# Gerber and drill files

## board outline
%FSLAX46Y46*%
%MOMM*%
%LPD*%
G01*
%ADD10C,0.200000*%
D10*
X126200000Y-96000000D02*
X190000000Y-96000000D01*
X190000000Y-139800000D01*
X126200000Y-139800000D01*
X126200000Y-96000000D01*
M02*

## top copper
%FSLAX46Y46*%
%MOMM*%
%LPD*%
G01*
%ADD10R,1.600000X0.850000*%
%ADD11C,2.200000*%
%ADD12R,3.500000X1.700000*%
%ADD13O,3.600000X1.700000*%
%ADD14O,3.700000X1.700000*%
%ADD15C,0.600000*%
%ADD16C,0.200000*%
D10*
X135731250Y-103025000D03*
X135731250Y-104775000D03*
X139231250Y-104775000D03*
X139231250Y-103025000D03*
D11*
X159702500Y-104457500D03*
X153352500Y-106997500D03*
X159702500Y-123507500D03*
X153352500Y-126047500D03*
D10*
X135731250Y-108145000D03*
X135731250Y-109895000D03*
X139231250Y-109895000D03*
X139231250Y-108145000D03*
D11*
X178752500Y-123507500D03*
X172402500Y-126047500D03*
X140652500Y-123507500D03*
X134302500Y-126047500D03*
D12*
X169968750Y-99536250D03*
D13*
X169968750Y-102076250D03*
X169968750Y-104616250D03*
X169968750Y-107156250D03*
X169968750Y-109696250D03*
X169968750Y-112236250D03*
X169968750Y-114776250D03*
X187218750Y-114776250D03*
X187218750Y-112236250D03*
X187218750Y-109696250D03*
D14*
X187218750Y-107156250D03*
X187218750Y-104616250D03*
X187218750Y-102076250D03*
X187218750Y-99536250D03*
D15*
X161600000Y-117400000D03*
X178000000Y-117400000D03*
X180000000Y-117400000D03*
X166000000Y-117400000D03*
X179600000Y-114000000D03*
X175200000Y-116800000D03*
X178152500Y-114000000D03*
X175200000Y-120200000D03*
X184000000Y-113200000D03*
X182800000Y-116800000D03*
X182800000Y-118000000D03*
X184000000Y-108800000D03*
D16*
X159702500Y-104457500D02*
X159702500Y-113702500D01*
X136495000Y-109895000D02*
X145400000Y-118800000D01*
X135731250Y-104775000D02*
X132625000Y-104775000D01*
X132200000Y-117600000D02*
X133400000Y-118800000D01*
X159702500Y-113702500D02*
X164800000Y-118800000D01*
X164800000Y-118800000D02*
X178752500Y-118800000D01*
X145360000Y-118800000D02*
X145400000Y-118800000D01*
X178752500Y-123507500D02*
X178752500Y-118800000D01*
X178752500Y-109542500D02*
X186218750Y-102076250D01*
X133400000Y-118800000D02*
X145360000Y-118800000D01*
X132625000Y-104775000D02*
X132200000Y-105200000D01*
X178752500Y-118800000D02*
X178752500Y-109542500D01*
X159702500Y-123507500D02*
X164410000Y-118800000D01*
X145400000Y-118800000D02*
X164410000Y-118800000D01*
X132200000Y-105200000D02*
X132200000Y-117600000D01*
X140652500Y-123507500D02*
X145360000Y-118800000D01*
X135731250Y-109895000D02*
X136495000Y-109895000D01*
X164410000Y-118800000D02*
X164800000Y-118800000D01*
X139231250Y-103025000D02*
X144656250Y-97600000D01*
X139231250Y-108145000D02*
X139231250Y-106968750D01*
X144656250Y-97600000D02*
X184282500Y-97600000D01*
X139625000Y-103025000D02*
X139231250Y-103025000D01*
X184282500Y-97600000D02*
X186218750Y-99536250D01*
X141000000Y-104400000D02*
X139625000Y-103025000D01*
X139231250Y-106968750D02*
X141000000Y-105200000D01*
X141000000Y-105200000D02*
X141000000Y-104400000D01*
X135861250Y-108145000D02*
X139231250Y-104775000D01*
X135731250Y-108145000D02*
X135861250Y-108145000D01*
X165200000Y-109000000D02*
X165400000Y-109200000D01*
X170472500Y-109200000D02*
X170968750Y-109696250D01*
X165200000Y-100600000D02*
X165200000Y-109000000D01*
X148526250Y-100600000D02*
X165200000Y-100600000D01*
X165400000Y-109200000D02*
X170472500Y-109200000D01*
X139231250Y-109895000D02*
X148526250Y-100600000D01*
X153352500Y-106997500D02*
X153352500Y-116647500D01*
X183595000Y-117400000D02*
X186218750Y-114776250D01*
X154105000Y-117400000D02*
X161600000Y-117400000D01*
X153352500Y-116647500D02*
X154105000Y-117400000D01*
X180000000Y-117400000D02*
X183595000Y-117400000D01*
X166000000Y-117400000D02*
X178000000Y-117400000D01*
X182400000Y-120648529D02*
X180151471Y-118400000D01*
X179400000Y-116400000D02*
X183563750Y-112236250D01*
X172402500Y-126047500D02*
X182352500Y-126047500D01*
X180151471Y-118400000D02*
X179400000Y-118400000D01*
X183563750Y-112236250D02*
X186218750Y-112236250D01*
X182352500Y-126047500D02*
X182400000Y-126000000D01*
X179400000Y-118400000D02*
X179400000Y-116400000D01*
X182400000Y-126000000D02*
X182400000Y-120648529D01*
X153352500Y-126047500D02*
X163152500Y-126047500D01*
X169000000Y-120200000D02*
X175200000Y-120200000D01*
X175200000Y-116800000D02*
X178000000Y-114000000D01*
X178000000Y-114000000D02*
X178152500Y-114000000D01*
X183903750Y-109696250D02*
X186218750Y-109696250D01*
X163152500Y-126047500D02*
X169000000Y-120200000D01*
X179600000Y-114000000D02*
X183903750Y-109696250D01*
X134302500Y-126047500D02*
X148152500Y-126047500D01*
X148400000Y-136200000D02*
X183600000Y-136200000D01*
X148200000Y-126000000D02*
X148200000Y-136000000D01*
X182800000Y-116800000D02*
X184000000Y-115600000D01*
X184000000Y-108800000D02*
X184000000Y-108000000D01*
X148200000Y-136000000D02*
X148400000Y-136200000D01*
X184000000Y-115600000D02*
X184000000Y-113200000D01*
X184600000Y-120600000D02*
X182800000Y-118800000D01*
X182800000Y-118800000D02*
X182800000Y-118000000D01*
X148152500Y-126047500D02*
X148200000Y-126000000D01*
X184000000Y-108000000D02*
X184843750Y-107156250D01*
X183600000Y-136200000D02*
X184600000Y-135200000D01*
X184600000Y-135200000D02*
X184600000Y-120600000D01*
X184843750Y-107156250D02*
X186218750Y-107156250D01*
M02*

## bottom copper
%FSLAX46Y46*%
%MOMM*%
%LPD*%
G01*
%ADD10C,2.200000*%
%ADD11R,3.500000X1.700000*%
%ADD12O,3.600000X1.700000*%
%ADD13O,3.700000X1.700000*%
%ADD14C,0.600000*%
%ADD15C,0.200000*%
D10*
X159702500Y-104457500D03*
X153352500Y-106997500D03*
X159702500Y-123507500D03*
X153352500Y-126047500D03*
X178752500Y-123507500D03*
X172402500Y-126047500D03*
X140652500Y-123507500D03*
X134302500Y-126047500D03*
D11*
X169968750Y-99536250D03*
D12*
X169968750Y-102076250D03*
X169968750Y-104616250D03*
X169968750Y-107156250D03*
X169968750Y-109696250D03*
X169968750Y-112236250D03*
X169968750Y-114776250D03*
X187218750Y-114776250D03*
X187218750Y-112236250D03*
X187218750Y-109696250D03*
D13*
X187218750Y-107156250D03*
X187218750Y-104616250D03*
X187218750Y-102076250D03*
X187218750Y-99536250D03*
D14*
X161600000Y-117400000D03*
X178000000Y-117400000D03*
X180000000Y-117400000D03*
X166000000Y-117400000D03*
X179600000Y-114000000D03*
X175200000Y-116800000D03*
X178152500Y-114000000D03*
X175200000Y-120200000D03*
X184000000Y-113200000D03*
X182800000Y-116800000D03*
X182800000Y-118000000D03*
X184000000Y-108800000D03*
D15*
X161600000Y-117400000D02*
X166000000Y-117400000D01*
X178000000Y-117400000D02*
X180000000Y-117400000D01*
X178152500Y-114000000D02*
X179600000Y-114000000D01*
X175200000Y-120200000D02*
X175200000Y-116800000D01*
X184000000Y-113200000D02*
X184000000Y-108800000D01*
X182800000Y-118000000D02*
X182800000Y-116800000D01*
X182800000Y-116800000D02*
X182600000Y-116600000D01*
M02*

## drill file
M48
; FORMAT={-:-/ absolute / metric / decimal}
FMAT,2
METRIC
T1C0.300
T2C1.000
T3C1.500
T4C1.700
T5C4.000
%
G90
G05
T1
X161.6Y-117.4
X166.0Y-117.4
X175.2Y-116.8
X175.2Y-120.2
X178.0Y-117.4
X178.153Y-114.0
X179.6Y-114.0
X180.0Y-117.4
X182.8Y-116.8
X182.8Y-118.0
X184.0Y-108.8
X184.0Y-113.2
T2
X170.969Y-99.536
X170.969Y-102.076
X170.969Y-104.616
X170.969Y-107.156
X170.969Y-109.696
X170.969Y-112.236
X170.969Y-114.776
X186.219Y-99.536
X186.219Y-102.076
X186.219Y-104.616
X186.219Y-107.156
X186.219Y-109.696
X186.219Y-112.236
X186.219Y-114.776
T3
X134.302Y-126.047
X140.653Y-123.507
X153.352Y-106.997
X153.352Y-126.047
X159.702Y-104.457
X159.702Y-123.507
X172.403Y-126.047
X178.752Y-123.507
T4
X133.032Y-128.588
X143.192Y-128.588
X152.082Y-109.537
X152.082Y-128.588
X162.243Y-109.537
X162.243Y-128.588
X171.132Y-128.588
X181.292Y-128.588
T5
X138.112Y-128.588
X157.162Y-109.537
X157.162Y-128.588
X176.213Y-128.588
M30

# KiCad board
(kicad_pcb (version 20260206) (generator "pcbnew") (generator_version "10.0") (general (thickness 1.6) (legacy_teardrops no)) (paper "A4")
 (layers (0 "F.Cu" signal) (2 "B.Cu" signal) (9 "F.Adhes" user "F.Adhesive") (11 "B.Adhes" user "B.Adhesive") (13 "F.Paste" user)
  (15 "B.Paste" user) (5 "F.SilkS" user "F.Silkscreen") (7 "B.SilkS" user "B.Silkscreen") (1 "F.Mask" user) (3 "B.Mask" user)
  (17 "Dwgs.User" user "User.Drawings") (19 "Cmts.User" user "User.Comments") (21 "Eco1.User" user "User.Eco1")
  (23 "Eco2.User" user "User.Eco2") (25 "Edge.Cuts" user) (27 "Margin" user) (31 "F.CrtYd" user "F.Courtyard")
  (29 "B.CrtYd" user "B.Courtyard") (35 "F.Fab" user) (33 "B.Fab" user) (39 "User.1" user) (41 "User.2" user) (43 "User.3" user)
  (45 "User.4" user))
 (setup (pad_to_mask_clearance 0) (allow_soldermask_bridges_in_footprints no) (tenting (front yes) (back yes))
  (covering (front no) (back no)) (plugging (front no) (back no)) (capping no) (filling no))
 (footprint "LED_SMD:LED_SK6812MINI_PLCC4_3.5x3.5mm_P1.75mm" (layer "F.Cu") (at 137.48125 103.9)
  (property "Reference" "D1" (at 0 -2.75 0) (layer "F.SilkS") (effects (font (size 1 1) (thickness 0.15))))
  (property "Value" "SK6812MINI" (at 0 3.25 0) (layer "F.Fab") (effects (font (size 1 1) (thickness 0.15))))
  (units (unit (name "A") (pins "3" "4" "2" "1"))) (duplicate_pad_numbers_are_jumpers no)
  (pad "1" smd rect (at -1.75 -0.875) (size 1.6 0.85) (layers "F.Cu" "F.Mask" "F.Paste") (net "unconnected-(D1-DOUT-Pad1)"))
  (pad "2" smd rect (at -1.75 0.875) (size 1.6 0.85) (layers "F.Cu" "F.Mask" "F.Paste") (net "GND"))
  (pad "3" smd rect (at 1.75 0.875) (size 1.6 0.85) (layers "F.Cu" "F.Mask" "F.Paste") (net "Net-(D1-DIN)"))
  (pad "4" smd rect (at 1.75 -0.875) (size 1.6 0.85) (layers "F.Cu" "F.Mask" "F.Paste") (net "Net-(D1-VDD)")))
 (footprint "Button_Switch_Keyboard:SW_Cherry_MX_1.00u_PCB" (layer "F.Cu") (at 159.7025 104.4575)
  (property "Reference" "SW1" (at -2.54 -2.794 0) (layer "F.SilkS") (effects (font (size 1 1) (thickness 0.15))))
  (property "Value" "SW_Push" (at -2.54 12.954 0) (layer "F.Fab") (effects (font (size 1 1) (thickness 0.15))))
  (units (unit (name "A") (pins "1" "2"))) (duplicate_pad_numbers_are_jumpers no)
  (pad "" np_thru_hole circle (at -7.62 5.08) (size 1.7 1.7) (drill 1.7) (layers "*.Cu" "*.Mask"))
  (pad "" np_thru_hole circle (at -2.54 5.08) (size 4 4) (drill 4) (layers "*.Cu" "*.Mask"))
  (pad "" np_thru_hole circle (at 2.54 5.08) (size 1.7 1.7) (drill 1.7) (layers "*.Cu" "*.Mask"))
  (pad "1" thru_hole circle (at 0 0) (size 2.2 2.2) (drill 1.5) (layers "*.Cu" "*.Mask") (remove_unused_layers no) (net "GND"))
  (pad "2" thru_hole circle (at -6.35 2.54) (size 2.2 2.2) (drill 1.5) (layers "*.Cu" "*.Mask") (remove_unused_layers no)
   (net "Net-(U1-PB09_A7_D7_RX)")))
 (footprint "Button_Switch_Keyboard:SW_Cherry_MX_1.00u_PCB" (layer "F.Cu") (at 159.7025 123.5075)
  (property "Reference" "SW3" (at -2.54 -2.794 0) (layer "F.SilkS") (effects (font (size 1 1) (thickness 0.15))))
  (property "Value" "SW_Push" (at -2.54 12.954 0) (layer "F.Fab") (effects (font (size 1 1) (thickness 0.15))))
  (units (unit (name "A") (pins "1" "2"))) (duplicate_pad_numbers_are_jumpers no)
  (pad "" np_thru_hole circle (at -7.62 5.08) (size 1.7 1.7) (drill 1.7) (layers "*.Cu" "*.Mask"))
  (pad "" np_thru_hole circle (at -2.54 5.08) (size 4 4) (drill 4) (layers "*.Cu" "*.Mask"))
  (pad "" np_thru_hole circle (at 2.54 5.08) (size 1.7 1.7) (drill 1.7) (layers "*.Cu" "*.Mask"))
  (pad "1" thru_hole circle (at 0 0) (size 2.2 2.2) (drill 1.5) (layers "*.Cu" "*.Mask") (remove_unused_layers no) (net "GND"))
  (pad "2" thru_hole circle (at -6.35 2.54) (size 2.2 2.2) (drill 1.5) (layers "*.Cu" "*.Mask") (remove_unused_layers no)
   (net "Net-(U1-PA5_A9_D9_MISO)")))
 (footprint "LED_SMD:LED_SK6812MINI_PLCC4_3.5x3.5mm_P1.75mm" (layer "F.Cu") (at 137.48125 109.02)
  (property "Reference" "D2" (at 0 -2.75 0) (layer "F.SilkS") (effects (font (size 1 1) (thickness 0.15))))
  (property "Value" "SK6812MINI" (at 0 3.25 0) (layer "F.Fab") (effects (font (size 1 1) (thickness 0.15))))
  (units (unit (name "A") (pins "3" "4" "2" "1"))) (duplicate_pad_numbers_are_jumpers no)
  (pad "1" smd rect (at -1.75 -0.875) (size 1.6 0.85) (layers "F.Cu" "F.Mask" "F.Paste") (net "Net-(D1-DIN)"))
  (pad "2" smd rect (at -1.75 0.875) (size 1.6 0.85) (layers "F.Cu" "F.Mask" "F.Paste") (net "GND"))
  (pad "3" smd rect (at 1.75 0.875) (size 1.6 0.85) (layers "F.Cu" "F.Mask" "F.Paste") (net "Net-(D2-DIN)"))
  (pad "4" smd rect (at 1.75 -0.875) (size 1.6 0.85) (layers "F.Cu" "F.Mask" "F.Paste") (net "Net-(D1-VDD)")))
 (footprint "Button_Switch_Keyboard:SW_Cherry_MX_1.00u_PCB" (layer "F.Cu") (at 178.7525 123.5075)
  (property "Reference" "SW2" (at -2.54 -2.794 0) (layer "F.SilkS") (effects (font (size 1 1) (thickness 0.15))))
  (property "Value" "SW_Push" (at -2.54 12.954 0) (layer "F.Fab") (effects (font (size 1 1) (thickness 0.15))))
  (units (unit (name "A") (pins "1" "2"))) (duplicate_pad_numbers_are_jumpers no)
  (pad "" np_thru_hole circle (at -7.62 5.08) (size 1.7 1.7) (drill 1.7) (layers "*.Cu" "*.Mask"))
  (pad "" np_thru_hole circle (at -2.54 5.08) (size 4 4) (drill 4) (layers "*.Cu" "*.Mask"))
  (pad "" np_thru_hole circle (at 2.54 5.08) (size 1.7 1.7) (drill 1.7) (layers "*.Cu" "*.Mask"))
  (pad "1" thru_hole circle (at 0 0) (size 2.2 2.2) (drill 1.5) (layers "*.Cu" "*.Mask") (remove_unused_layers no) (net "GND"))
  (pad "2" thru_hole circle (at -6.35 2.54) (size 2.2 2.2) (drill 1.5) (layers "*.Cu" "*.Mask") (remove_unused_layers no)
   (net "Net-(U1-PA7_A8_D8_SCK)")))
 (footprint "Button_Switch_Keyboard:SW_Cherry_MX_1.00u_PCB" (layer "F.Cu") (at 140.6525 123.5075)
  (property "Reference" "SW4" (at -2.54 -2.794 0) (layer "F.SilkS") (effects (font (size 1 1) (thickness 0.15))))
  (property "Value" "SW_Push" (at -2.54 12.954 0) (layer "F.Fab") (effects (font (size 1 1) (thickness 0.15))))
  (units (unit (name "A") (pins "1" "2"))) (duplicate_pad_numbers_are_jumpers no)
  (pad "" np_thru_hole circle (at -7.62 5.08) (size 1.7 1.7) (drill 1.7) (layers "*.Cu" "*.Mask"))
  (pad "" np_thru_hole circle (at -2.54 5.08) (size 4 4) (drill 4) (layers "*.Cu" "*.Mask"))
  (pad "" np_thru_hole circle (at 2.54 5.08) (size 1.7 1.7) (drill 1.7) (layers "*.Cu" "*.Mask"))
  (pad "1" thru_hole circle (at 0 0) (size 2.2 2.2) (drill 1.5) (layers "*.Cu" "*.Mask") (remove_unused_layers no) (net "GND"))
  (pad "2" thru_hole circle (at -6.35 2.54) (size 2.2 2.2) (drill 1.5) (layers "*.Cu" "*.Mask") (remove_unused_layers no)
   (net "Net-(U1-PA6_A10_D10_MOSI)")))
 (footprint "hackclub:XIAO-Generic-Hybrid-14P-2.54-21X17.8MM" (layer "F.Cu") (at 178.59375 107.15625)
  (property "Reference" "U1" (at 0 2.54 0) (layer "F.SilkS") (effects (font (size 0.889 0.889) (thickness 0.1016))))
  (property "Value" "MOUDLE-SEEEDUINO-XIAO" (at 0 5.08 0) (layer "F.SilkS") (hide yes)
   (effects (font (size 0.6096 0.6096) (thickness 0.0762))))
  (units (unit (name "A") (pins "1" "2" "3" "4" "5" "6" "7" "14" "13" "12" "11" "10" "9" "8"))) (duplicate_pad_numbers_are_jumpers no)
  (pad "1" thru_hole rect (at -7.625 -7.62) (size 3.5 1.7) (drill 1 (offset -1 0)) (layers "*.Cu" "*.Mask") (remove_unused_layers no)
   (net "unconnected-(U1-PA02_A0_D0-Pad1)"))
  (pad "2" thru_hole oval (at -7.625 -5.08) (size 3.6 1.7) (drill 1 (offset -1 0)) (layers "*.Cu" "*.Mask") (remove_unused_layers no)
   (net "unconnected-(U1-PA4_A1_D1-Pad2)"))
  (pad "3" thru_hole oval (at -7.625 -2.54) (size 3.6 1.7) (drill 1 (offset -1 0)) (layers "*.Cu" "*.Mask") (remove_unused_layers no)
   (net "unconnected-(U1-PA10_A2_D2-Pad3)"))
  (pad "4" thru_hole oval (at -7.625 0) (size 3.6 1.7) (drill 1 (offset -1 0)) (layers "*.Cu" "*.Mask") (remove_unused_layers no)
   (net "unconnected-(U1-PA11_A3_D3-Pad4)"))
  (pad "5" thru_hole oval (at -7.625 2.54) (size 3.6 1.7) (drill 1 (offset -1 0)) (layers "*.Cu" "*.Mask") (remove_unused_layers no)
   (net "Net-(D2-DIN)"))
  (pad "6" thru_hole oval (at -7.625 5.08 180) (size 3.6 1.7) (drill 1 (offset 1 0)) (layers "*.Cu" "*.Mask") (remove_unused_layers no)
   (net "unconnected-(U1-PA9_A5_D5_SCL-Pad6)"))
  (pad "7" thru_hole oval (at -7.625 7.62) (size 3.6 1.7) (drill 1 (offset -1 0)) (layers "*.Cu" "*.Mask") (remove_unused_layers no)
   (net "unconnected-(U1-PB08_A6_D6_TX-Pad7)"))
  (pad "8" thru_hole oval (at 7.625 7.62) (size 3.6 1.7) (drill 1 (offset 1 0)) (layers "*.Cu" "*.Mask") (remove_unused_layers no)
   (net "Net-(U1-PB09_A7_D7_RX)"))
  (pad "9" thru_hole oval (at 7.625 5.08) (size 3.6 1.7) (drill 1 (offset 1 0)) (layers "*.Cu" "*.Mask") (remove_unused_layers no)
   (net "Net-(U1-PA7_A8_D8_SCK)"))
  (pad "10" thru_hole oval (at 7.625 2.54) (size 3.6 1.7) (drill 1 (offset 1 0)) (layers "*.Cu" "*.Mask") (remove_unused_layers no)
   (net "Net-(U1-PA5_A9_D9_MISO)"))
  (pad "11" thru_hole oval (at 7.625 0) (size 3.7 1.7) (drill 1 (offset 1 0)) (layers "*.Cu" "*.Mask") (remove_unused_layers no)
   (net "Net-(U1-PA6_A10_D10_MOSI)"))
  (pad "12" thru_hole oval (at 7.625 -2.54) (size 3.7 1.7) (drill 1 (offset 1 0)) (layers "*.Cu" "*.Mask") (remove_unused_layers no)
   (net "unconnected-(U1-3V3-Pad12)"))
  (pad "13" thru_hole oval (at 7.625 -5.08) (size 3.7 1.7) (drill 1 (offset 1 0)) (layers "*.Cu" "*.Mask") (remove_unused_layers no)
   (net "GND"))
  (pad "14" thru_hole oval (at 7.625 -7.62) (size 3.7 1.7) (drill 1 (offset 1 0)) (layers "*.Cu" "*.Mask") (remove_unused_layers no)
   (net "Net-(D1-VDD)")))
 (gr_rect (start 126.2 96) (end 190 139.8) (stroke (width 0.2) (type solid)) (fill no) (layer "Edge.Cuts"))
 (segment (start 159.7025 104.4575) (end 159.7025 113.7025) (width 0.2) (layer "F.Cu") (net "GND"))
 (segment (start 136.495 109.895) (end 145.4 118.8) (width 0.2) (layer "F.Cu") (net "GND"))
 (segment (start 135.73125 104.775) (end 132.625 104.775) (width 0.2) (layer "F.Cu") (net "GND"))
 (segment (start 132.2 117.6) (end 133.4 118.8) (width 0.2) (layer "F.Cu") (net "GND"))
 (segment (start 159.7025 113.7025) (end 164.8 118.8) (width 0.2) (layer "F.Cu") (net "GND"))
 (segment (start 164.8 118.8) (end 178.7525 118.8) (width 0.2) (layer "F.Cu") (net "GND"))
 (segment (start 145.36 118.8) (end 145.4 118.8) (width 0.2) (layer "F.Cu") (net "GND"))
 (segment (start 178.7525 123.5075) (end 178.7525 118.8) (width 0.2) (layer "F.Cu") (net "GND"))
 (segment (start 178.7525 109.5425) (end 186.21875 102.07625) (width 0.2) (layer "F.Cu") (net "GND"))
 (segment (start 133.4 118.8) (end 145.36 118.8) (width 0.2) (layer "F.Cu") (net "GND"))
 (segment (start 132.625 104.775) (end 132.2 105.2) (width 0.2) (layer "F.Cu") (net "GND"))
 (segment (start 178.7525 118.8) (end 178.7525 109.5425) (width 0.2) (layer "F.Cu") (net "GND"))
 (segment (start 159.7025 123.5075) (end 164.41 118.8) (width 0.2) (layer "F.Cu") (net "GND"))
 (segment (start 145.4 118.8) (end 164.41 118.8) (width 0.2) (layer "F.Cu") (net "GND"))
 (segment (start 132.2 105.2) (end 132.2 117.6) (width 0.2) (layer "F.Cu") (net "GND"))
 (segment (start 140.6525 123.5075) (end 145.36 118.8) (width 0.2) (layer "F.Cu") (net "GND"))
 (segment (start 135.73125 109.895) (end 136.495 109.895) (width 0.2) (layer "F.Cu") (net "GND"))
 (segment (start 164.41 118.8) (end 164.8 118.8) (width 0.2) (layer "F.Cu") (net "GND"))
 (segment (start 139.23125 103.025) (end 144.65625 97.6) (width 0.2) (layer "F.Cu") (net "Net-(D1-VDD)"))
 (segment (start 139.23125 108.145) (end 139.23125 106.96875) (width 0.2) (layer "F.Cu") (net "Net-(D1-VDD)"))
 (segment (start 144.65625 97.6) (end 184.2825 97.6) (width 0.2) (layer "F.Cu") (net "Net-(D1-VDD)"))
 (segment (start 139.625 103.025) (end 139.23125 103.025) (width 0.2) (layer "F.Cu") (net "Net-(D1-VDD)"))
 (segment (start 184.2825 97.6) (end 186.21875 99.53625) (width 0.2) (layer "F.Cu") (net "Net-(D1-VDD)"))
 (segment (start 141 104.4) (end 139.625 103.025) (width 0.2) (layer "F.Cu") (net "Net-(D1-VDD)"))
 (segment (start 139.23125 106.96875) (end 141 105.2) (width 0.2) (layer "F.Cu") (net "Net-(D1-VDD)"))
 (segment (start 141 105.2) (end 141 104.4) (width 0.2) (layer "F.Cu") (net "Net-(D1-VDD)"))
 (segment (start 135.86125 108.145) (end 139.23125 104.775) (width 0.2) (layer "F.Cu") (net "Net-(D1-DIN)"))
 (segment (start 135.73125 108.145) (end 135.86125 108.145) (width 0.2) (layer "F.Cu") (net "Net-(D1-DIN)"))
 (segment (start 165.2 109) (end 165.4 109.2) (width 0.2) (layer "F.Cu") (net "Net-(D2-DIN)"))
 (segment (start 170.4725 109.2) (end 170.96875 109.69625) (width 0.2) (layer "F.Cu") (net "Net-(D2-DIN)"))
 (segment (start 165.2 100.6) (end 165.2 109) (width 0.2) (layer "F.Cu") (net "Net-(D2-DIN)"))
 (segment (start 148.52625 100.6) (end 165.2 100.6) (width 0.2) (layer "F.Cu") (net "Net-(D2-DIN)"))
 (segment (start 165.4 109.2) (end 170.4725 109.2) (width 0.2) (layer "F.Cu") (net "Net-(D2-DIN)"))
 (segment (start 139.23125 109.895) (end 148.52625 100.6) (width 0.2) (layer "F.Cu") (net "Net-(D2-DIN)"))
 (segment (start 153.3525 106.9975) (end 153.3525 116.6475) (width 0.2) (layer "F.Cu") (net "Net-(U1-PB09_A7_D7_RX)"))
 (segment (start 183.595 117.4) (end 186.21875 114.77625) (width 0.2) (layer "F.Cu") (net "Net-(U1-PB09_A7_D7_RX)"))
 (segment (start 154.105 117.4) (end 161.6 117.4) (width 0.2) (layer "F.Cu") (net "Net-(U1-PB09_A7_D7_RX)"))
 (segment (start 153.3525 116.6475) (end 154.105 117.4) (width 0.2) (layer "F.Cu") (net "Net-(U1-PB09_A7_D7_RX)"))
 (segment (start 180 117.4) (end 183.595 117.4) (width 0.2) (layer "F.Cu") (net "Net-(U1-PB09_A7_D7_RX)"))
 (segment (start 166 117.4) (end 178 117.4) (width 0.2) (layer "F.Cu") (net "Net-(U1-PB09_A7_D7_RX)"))
 (via (at 161.6 117.4) (size 0.6) (drill 0.3) (layers "F.Cu" "B.Cu") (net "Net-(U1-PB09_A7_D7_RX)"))
 (via (at 178 117.4) (size 0.6) (drill 0.3) (layers "F.Cu" "B.Cu") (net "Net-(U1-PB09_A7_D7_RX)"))
 (via (at 180 117.4) (size 0.6) (drill 0.3) (layers "F.Cu" "B.Cu") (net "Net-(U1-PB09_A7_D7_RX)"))
 (via (at 166 117.4) (size 0.6) (drill 0.3) (layers "F.Cu" "B.Cu") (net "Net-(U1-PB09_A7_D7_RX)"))
 (segment (start 161.6 117.4) (end 166 117.4) (width 0.2) (layer "B.Cu") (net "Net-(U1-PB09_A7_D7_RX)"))
 (segment (start 178 117.4) (end 180 117.4) (width 0.2) (layer "B.Cu") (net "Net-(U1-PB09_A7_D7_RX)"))
 (segment (start 182.4 120.648529) (end 180.151471 118.4) (width 0.2) (layer "F.Cu") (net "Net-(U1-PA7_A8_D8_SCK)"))
 (segment (start 179.4 116.4) (end 183.56375 112.23625) (width 0.2) (layer "F.Cu") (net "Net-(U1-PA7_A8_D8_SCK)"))
 (segment (start 172.4025 126.0475) (end 182.3525 126.0475) (width 0.2) (layer "F.Cu") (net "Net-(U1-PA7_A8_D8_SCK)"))
 (segment (start 180.151471 118.4) (end 179.4 118.4) (width 0.2) (layer "F.Cu") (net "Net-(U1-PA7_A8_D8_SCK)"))
 (segment (start 183.56375 112.23625) (end 186.21875 112.23625) (width 0.2) (layer "F.Cu") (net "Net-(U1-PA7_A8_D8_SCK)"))
 (segment (start 182.3525 126.0475) (end 182.4 126) (width 0.2) (layer "F.Cu") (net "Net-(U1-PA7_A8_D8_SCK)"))
 (segment (start 179.4 118.4) (end 179.4 116.4) (width 0.2) (layer "F.Cu") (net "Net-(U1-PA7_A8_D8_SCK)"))
 (segment (start 182.4 126) (end 182.4 120.648529) (width 0.2) (layer "F.Cu") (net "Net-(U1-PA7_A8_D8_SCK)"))
 (segment (start 153.3525 126.0475) (end 163.1525 126.0475) (width 0.2) (layer "F.Cu") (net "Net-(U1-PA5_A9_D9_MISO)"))
 (segment (start 169 120.2) (end 175.2 120.2) (width 0.2) (layer "F.Cu") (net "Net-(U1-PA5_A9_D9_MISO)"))
 (segment (start 175.2 116.8) (end 178 114) (width 0.2) (layer "F.Cu") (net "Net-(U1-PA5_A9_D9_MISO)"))
 (segment (start 178 114) (end 178.1525 114) (width 0.2) (layer "F.Cu") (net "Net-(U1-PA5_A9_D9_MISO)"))
 (segment (start 183.90375 109.69625) (end 186.21875 109.69625) (width 0.2) (layer "F.Cu") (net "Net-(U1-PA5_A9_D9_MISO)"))
 (segment (start 163.1525 126.0475) (end 169 120.2) (width 0.2) (layer "F.Cu") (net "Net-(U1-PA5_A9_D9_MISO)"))
 (segment (start 179.6 114) (end 183.90375 109.69625) (width 0.2) (layer "F.Cu") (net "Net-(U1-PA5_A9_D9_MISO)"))
 (via (at 179.6 114) (size 0.6) (drill 0.3) (layers "F.Cu" "B.Cu") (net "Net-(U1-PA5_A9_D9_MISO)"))
 (via (at 175.2 116.8) (size 0.6) (drill 0.3) (layers "F.Cu" "B.Cu") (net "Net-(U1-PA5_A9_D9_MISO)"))
 (via (at 178.1525 114) (size 0.6) (drill 0.3) (layers "F.Cu" "B.Cu") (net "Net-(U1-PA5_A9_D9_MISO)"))
 (via (at 175.2 120.2) (size 0.6) (drill 0.3) (layers "F.Cu" "B.Cu") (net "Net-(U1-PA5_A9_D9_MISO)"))
 (segment (start 178.1525 114) (end 179.6 114) (width 0.2) (layer "B.Cu") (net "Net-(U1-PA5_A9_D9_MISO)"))
 (segment (start 175.2 120.2) (end 175.2 116.8) (width 0.2) (layer "B.Cu") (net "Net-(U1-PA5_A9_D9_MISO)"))
 (segment (start 134.3025 126.0475) (end 148.1525 126.0475) (width 0.2) (layer "F.Cu") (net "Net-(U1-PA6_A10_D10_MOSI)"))
 (segment (start 148.4 136.2) (end 183.6 136.2) (width 0.2) (layer "F.Cu") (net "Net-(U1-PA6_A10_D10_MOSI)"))
 (segment (start 148.2 126) (end 148.2 136) (width 0.2) (layer "F.Cu") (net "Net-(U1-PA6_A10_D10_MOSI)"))
 (segment (start 182.8 116.8) (end 184 115.6) (width 0.2) (layer "F.Cu") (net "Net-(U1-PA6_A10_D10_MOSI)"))
 (segment (start 184 108.8) (end 184 108) (width 0.2) (layer "F.Cu") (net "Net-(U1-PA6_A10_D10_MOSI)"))
 (segment (start 148.2 136) (end 148.4 136.2) (width 0.2) (layer "F.Cu") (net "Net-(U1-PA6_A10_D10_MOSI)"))
 (segment (start 184 115.6) (end 184 113.2) (width 0.2) (layer "F.Cu") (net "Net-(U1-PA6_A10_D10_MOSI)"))
 (segment (start 184.6 120.6) (end 182.8 118.8) (width 0.2) (layer "F.Cu") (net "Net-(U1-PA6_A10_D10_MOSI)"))
 (segment (start 182.8 118.8) (end 182.8 118) (width 0.2) (layer "F.Cu") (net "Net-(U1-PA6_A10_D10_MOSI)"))
 (segment (start 148.1525 126.0475) (end 148.2 126) (width 0.2) (layer "F.Cu") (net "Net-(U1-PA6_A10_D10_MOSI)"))
 (segment (start 184 108) (end 184.84375 107.15625) (width 0.2) (layer "F.Cu") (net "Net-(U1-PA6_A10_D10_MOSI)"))
 (segment (start 183.6 136.2) (end 184.6 135.2) (width 0.2) (layer "F.Cu") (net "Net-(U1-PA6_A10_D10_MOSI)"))
 (segment (start 184.6 135.2) (end 184.6 120.6) (width 0.2) (layer "F.Cu") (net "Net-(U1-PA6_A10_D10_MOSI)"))
 (segment (start 184.84375 107.15625) (end 186.21875 107.15625) (width 0.2) (layer "F.Cu") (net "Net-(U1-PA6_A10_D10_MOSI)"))
 (via (at 184 113.2) (size 0.6) (drill 0.3) (layers "F.Cu" "B.Cu") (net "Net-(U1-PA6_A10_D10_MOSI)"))
 (via (at 182.8 116.8) (size 0.6) (drill 0.3) (layers "F.Cu" "B.Cu") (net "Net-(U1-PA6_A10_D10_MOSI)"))
 (via (at 182.8 118) (size 0.6) (drill 0.3) (layers "F.Cu" "B.Cu") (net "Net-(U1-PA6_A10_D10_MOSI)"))
 (via (at 184 108.8) (size 0.6) (drill 0.3) (layers "F.Cu" "B.Cu") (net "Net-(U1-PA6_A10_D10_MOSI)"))
 (segment (start 184 113.2) (end 184 108.8) (width 0.2) (layer "B.Cu") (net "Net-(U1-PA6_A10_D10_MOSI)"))
 (segment (start 182.8 118) (end 182.8 116.8) (width 0.2) (layer "B.Cu") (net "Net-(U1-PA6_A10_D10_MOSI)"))
 (segment (start 182.8 116.8) (end 182.6 116.6) (width 0.2) (layer "B.Cu") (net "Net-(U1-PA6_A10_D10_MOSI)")))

